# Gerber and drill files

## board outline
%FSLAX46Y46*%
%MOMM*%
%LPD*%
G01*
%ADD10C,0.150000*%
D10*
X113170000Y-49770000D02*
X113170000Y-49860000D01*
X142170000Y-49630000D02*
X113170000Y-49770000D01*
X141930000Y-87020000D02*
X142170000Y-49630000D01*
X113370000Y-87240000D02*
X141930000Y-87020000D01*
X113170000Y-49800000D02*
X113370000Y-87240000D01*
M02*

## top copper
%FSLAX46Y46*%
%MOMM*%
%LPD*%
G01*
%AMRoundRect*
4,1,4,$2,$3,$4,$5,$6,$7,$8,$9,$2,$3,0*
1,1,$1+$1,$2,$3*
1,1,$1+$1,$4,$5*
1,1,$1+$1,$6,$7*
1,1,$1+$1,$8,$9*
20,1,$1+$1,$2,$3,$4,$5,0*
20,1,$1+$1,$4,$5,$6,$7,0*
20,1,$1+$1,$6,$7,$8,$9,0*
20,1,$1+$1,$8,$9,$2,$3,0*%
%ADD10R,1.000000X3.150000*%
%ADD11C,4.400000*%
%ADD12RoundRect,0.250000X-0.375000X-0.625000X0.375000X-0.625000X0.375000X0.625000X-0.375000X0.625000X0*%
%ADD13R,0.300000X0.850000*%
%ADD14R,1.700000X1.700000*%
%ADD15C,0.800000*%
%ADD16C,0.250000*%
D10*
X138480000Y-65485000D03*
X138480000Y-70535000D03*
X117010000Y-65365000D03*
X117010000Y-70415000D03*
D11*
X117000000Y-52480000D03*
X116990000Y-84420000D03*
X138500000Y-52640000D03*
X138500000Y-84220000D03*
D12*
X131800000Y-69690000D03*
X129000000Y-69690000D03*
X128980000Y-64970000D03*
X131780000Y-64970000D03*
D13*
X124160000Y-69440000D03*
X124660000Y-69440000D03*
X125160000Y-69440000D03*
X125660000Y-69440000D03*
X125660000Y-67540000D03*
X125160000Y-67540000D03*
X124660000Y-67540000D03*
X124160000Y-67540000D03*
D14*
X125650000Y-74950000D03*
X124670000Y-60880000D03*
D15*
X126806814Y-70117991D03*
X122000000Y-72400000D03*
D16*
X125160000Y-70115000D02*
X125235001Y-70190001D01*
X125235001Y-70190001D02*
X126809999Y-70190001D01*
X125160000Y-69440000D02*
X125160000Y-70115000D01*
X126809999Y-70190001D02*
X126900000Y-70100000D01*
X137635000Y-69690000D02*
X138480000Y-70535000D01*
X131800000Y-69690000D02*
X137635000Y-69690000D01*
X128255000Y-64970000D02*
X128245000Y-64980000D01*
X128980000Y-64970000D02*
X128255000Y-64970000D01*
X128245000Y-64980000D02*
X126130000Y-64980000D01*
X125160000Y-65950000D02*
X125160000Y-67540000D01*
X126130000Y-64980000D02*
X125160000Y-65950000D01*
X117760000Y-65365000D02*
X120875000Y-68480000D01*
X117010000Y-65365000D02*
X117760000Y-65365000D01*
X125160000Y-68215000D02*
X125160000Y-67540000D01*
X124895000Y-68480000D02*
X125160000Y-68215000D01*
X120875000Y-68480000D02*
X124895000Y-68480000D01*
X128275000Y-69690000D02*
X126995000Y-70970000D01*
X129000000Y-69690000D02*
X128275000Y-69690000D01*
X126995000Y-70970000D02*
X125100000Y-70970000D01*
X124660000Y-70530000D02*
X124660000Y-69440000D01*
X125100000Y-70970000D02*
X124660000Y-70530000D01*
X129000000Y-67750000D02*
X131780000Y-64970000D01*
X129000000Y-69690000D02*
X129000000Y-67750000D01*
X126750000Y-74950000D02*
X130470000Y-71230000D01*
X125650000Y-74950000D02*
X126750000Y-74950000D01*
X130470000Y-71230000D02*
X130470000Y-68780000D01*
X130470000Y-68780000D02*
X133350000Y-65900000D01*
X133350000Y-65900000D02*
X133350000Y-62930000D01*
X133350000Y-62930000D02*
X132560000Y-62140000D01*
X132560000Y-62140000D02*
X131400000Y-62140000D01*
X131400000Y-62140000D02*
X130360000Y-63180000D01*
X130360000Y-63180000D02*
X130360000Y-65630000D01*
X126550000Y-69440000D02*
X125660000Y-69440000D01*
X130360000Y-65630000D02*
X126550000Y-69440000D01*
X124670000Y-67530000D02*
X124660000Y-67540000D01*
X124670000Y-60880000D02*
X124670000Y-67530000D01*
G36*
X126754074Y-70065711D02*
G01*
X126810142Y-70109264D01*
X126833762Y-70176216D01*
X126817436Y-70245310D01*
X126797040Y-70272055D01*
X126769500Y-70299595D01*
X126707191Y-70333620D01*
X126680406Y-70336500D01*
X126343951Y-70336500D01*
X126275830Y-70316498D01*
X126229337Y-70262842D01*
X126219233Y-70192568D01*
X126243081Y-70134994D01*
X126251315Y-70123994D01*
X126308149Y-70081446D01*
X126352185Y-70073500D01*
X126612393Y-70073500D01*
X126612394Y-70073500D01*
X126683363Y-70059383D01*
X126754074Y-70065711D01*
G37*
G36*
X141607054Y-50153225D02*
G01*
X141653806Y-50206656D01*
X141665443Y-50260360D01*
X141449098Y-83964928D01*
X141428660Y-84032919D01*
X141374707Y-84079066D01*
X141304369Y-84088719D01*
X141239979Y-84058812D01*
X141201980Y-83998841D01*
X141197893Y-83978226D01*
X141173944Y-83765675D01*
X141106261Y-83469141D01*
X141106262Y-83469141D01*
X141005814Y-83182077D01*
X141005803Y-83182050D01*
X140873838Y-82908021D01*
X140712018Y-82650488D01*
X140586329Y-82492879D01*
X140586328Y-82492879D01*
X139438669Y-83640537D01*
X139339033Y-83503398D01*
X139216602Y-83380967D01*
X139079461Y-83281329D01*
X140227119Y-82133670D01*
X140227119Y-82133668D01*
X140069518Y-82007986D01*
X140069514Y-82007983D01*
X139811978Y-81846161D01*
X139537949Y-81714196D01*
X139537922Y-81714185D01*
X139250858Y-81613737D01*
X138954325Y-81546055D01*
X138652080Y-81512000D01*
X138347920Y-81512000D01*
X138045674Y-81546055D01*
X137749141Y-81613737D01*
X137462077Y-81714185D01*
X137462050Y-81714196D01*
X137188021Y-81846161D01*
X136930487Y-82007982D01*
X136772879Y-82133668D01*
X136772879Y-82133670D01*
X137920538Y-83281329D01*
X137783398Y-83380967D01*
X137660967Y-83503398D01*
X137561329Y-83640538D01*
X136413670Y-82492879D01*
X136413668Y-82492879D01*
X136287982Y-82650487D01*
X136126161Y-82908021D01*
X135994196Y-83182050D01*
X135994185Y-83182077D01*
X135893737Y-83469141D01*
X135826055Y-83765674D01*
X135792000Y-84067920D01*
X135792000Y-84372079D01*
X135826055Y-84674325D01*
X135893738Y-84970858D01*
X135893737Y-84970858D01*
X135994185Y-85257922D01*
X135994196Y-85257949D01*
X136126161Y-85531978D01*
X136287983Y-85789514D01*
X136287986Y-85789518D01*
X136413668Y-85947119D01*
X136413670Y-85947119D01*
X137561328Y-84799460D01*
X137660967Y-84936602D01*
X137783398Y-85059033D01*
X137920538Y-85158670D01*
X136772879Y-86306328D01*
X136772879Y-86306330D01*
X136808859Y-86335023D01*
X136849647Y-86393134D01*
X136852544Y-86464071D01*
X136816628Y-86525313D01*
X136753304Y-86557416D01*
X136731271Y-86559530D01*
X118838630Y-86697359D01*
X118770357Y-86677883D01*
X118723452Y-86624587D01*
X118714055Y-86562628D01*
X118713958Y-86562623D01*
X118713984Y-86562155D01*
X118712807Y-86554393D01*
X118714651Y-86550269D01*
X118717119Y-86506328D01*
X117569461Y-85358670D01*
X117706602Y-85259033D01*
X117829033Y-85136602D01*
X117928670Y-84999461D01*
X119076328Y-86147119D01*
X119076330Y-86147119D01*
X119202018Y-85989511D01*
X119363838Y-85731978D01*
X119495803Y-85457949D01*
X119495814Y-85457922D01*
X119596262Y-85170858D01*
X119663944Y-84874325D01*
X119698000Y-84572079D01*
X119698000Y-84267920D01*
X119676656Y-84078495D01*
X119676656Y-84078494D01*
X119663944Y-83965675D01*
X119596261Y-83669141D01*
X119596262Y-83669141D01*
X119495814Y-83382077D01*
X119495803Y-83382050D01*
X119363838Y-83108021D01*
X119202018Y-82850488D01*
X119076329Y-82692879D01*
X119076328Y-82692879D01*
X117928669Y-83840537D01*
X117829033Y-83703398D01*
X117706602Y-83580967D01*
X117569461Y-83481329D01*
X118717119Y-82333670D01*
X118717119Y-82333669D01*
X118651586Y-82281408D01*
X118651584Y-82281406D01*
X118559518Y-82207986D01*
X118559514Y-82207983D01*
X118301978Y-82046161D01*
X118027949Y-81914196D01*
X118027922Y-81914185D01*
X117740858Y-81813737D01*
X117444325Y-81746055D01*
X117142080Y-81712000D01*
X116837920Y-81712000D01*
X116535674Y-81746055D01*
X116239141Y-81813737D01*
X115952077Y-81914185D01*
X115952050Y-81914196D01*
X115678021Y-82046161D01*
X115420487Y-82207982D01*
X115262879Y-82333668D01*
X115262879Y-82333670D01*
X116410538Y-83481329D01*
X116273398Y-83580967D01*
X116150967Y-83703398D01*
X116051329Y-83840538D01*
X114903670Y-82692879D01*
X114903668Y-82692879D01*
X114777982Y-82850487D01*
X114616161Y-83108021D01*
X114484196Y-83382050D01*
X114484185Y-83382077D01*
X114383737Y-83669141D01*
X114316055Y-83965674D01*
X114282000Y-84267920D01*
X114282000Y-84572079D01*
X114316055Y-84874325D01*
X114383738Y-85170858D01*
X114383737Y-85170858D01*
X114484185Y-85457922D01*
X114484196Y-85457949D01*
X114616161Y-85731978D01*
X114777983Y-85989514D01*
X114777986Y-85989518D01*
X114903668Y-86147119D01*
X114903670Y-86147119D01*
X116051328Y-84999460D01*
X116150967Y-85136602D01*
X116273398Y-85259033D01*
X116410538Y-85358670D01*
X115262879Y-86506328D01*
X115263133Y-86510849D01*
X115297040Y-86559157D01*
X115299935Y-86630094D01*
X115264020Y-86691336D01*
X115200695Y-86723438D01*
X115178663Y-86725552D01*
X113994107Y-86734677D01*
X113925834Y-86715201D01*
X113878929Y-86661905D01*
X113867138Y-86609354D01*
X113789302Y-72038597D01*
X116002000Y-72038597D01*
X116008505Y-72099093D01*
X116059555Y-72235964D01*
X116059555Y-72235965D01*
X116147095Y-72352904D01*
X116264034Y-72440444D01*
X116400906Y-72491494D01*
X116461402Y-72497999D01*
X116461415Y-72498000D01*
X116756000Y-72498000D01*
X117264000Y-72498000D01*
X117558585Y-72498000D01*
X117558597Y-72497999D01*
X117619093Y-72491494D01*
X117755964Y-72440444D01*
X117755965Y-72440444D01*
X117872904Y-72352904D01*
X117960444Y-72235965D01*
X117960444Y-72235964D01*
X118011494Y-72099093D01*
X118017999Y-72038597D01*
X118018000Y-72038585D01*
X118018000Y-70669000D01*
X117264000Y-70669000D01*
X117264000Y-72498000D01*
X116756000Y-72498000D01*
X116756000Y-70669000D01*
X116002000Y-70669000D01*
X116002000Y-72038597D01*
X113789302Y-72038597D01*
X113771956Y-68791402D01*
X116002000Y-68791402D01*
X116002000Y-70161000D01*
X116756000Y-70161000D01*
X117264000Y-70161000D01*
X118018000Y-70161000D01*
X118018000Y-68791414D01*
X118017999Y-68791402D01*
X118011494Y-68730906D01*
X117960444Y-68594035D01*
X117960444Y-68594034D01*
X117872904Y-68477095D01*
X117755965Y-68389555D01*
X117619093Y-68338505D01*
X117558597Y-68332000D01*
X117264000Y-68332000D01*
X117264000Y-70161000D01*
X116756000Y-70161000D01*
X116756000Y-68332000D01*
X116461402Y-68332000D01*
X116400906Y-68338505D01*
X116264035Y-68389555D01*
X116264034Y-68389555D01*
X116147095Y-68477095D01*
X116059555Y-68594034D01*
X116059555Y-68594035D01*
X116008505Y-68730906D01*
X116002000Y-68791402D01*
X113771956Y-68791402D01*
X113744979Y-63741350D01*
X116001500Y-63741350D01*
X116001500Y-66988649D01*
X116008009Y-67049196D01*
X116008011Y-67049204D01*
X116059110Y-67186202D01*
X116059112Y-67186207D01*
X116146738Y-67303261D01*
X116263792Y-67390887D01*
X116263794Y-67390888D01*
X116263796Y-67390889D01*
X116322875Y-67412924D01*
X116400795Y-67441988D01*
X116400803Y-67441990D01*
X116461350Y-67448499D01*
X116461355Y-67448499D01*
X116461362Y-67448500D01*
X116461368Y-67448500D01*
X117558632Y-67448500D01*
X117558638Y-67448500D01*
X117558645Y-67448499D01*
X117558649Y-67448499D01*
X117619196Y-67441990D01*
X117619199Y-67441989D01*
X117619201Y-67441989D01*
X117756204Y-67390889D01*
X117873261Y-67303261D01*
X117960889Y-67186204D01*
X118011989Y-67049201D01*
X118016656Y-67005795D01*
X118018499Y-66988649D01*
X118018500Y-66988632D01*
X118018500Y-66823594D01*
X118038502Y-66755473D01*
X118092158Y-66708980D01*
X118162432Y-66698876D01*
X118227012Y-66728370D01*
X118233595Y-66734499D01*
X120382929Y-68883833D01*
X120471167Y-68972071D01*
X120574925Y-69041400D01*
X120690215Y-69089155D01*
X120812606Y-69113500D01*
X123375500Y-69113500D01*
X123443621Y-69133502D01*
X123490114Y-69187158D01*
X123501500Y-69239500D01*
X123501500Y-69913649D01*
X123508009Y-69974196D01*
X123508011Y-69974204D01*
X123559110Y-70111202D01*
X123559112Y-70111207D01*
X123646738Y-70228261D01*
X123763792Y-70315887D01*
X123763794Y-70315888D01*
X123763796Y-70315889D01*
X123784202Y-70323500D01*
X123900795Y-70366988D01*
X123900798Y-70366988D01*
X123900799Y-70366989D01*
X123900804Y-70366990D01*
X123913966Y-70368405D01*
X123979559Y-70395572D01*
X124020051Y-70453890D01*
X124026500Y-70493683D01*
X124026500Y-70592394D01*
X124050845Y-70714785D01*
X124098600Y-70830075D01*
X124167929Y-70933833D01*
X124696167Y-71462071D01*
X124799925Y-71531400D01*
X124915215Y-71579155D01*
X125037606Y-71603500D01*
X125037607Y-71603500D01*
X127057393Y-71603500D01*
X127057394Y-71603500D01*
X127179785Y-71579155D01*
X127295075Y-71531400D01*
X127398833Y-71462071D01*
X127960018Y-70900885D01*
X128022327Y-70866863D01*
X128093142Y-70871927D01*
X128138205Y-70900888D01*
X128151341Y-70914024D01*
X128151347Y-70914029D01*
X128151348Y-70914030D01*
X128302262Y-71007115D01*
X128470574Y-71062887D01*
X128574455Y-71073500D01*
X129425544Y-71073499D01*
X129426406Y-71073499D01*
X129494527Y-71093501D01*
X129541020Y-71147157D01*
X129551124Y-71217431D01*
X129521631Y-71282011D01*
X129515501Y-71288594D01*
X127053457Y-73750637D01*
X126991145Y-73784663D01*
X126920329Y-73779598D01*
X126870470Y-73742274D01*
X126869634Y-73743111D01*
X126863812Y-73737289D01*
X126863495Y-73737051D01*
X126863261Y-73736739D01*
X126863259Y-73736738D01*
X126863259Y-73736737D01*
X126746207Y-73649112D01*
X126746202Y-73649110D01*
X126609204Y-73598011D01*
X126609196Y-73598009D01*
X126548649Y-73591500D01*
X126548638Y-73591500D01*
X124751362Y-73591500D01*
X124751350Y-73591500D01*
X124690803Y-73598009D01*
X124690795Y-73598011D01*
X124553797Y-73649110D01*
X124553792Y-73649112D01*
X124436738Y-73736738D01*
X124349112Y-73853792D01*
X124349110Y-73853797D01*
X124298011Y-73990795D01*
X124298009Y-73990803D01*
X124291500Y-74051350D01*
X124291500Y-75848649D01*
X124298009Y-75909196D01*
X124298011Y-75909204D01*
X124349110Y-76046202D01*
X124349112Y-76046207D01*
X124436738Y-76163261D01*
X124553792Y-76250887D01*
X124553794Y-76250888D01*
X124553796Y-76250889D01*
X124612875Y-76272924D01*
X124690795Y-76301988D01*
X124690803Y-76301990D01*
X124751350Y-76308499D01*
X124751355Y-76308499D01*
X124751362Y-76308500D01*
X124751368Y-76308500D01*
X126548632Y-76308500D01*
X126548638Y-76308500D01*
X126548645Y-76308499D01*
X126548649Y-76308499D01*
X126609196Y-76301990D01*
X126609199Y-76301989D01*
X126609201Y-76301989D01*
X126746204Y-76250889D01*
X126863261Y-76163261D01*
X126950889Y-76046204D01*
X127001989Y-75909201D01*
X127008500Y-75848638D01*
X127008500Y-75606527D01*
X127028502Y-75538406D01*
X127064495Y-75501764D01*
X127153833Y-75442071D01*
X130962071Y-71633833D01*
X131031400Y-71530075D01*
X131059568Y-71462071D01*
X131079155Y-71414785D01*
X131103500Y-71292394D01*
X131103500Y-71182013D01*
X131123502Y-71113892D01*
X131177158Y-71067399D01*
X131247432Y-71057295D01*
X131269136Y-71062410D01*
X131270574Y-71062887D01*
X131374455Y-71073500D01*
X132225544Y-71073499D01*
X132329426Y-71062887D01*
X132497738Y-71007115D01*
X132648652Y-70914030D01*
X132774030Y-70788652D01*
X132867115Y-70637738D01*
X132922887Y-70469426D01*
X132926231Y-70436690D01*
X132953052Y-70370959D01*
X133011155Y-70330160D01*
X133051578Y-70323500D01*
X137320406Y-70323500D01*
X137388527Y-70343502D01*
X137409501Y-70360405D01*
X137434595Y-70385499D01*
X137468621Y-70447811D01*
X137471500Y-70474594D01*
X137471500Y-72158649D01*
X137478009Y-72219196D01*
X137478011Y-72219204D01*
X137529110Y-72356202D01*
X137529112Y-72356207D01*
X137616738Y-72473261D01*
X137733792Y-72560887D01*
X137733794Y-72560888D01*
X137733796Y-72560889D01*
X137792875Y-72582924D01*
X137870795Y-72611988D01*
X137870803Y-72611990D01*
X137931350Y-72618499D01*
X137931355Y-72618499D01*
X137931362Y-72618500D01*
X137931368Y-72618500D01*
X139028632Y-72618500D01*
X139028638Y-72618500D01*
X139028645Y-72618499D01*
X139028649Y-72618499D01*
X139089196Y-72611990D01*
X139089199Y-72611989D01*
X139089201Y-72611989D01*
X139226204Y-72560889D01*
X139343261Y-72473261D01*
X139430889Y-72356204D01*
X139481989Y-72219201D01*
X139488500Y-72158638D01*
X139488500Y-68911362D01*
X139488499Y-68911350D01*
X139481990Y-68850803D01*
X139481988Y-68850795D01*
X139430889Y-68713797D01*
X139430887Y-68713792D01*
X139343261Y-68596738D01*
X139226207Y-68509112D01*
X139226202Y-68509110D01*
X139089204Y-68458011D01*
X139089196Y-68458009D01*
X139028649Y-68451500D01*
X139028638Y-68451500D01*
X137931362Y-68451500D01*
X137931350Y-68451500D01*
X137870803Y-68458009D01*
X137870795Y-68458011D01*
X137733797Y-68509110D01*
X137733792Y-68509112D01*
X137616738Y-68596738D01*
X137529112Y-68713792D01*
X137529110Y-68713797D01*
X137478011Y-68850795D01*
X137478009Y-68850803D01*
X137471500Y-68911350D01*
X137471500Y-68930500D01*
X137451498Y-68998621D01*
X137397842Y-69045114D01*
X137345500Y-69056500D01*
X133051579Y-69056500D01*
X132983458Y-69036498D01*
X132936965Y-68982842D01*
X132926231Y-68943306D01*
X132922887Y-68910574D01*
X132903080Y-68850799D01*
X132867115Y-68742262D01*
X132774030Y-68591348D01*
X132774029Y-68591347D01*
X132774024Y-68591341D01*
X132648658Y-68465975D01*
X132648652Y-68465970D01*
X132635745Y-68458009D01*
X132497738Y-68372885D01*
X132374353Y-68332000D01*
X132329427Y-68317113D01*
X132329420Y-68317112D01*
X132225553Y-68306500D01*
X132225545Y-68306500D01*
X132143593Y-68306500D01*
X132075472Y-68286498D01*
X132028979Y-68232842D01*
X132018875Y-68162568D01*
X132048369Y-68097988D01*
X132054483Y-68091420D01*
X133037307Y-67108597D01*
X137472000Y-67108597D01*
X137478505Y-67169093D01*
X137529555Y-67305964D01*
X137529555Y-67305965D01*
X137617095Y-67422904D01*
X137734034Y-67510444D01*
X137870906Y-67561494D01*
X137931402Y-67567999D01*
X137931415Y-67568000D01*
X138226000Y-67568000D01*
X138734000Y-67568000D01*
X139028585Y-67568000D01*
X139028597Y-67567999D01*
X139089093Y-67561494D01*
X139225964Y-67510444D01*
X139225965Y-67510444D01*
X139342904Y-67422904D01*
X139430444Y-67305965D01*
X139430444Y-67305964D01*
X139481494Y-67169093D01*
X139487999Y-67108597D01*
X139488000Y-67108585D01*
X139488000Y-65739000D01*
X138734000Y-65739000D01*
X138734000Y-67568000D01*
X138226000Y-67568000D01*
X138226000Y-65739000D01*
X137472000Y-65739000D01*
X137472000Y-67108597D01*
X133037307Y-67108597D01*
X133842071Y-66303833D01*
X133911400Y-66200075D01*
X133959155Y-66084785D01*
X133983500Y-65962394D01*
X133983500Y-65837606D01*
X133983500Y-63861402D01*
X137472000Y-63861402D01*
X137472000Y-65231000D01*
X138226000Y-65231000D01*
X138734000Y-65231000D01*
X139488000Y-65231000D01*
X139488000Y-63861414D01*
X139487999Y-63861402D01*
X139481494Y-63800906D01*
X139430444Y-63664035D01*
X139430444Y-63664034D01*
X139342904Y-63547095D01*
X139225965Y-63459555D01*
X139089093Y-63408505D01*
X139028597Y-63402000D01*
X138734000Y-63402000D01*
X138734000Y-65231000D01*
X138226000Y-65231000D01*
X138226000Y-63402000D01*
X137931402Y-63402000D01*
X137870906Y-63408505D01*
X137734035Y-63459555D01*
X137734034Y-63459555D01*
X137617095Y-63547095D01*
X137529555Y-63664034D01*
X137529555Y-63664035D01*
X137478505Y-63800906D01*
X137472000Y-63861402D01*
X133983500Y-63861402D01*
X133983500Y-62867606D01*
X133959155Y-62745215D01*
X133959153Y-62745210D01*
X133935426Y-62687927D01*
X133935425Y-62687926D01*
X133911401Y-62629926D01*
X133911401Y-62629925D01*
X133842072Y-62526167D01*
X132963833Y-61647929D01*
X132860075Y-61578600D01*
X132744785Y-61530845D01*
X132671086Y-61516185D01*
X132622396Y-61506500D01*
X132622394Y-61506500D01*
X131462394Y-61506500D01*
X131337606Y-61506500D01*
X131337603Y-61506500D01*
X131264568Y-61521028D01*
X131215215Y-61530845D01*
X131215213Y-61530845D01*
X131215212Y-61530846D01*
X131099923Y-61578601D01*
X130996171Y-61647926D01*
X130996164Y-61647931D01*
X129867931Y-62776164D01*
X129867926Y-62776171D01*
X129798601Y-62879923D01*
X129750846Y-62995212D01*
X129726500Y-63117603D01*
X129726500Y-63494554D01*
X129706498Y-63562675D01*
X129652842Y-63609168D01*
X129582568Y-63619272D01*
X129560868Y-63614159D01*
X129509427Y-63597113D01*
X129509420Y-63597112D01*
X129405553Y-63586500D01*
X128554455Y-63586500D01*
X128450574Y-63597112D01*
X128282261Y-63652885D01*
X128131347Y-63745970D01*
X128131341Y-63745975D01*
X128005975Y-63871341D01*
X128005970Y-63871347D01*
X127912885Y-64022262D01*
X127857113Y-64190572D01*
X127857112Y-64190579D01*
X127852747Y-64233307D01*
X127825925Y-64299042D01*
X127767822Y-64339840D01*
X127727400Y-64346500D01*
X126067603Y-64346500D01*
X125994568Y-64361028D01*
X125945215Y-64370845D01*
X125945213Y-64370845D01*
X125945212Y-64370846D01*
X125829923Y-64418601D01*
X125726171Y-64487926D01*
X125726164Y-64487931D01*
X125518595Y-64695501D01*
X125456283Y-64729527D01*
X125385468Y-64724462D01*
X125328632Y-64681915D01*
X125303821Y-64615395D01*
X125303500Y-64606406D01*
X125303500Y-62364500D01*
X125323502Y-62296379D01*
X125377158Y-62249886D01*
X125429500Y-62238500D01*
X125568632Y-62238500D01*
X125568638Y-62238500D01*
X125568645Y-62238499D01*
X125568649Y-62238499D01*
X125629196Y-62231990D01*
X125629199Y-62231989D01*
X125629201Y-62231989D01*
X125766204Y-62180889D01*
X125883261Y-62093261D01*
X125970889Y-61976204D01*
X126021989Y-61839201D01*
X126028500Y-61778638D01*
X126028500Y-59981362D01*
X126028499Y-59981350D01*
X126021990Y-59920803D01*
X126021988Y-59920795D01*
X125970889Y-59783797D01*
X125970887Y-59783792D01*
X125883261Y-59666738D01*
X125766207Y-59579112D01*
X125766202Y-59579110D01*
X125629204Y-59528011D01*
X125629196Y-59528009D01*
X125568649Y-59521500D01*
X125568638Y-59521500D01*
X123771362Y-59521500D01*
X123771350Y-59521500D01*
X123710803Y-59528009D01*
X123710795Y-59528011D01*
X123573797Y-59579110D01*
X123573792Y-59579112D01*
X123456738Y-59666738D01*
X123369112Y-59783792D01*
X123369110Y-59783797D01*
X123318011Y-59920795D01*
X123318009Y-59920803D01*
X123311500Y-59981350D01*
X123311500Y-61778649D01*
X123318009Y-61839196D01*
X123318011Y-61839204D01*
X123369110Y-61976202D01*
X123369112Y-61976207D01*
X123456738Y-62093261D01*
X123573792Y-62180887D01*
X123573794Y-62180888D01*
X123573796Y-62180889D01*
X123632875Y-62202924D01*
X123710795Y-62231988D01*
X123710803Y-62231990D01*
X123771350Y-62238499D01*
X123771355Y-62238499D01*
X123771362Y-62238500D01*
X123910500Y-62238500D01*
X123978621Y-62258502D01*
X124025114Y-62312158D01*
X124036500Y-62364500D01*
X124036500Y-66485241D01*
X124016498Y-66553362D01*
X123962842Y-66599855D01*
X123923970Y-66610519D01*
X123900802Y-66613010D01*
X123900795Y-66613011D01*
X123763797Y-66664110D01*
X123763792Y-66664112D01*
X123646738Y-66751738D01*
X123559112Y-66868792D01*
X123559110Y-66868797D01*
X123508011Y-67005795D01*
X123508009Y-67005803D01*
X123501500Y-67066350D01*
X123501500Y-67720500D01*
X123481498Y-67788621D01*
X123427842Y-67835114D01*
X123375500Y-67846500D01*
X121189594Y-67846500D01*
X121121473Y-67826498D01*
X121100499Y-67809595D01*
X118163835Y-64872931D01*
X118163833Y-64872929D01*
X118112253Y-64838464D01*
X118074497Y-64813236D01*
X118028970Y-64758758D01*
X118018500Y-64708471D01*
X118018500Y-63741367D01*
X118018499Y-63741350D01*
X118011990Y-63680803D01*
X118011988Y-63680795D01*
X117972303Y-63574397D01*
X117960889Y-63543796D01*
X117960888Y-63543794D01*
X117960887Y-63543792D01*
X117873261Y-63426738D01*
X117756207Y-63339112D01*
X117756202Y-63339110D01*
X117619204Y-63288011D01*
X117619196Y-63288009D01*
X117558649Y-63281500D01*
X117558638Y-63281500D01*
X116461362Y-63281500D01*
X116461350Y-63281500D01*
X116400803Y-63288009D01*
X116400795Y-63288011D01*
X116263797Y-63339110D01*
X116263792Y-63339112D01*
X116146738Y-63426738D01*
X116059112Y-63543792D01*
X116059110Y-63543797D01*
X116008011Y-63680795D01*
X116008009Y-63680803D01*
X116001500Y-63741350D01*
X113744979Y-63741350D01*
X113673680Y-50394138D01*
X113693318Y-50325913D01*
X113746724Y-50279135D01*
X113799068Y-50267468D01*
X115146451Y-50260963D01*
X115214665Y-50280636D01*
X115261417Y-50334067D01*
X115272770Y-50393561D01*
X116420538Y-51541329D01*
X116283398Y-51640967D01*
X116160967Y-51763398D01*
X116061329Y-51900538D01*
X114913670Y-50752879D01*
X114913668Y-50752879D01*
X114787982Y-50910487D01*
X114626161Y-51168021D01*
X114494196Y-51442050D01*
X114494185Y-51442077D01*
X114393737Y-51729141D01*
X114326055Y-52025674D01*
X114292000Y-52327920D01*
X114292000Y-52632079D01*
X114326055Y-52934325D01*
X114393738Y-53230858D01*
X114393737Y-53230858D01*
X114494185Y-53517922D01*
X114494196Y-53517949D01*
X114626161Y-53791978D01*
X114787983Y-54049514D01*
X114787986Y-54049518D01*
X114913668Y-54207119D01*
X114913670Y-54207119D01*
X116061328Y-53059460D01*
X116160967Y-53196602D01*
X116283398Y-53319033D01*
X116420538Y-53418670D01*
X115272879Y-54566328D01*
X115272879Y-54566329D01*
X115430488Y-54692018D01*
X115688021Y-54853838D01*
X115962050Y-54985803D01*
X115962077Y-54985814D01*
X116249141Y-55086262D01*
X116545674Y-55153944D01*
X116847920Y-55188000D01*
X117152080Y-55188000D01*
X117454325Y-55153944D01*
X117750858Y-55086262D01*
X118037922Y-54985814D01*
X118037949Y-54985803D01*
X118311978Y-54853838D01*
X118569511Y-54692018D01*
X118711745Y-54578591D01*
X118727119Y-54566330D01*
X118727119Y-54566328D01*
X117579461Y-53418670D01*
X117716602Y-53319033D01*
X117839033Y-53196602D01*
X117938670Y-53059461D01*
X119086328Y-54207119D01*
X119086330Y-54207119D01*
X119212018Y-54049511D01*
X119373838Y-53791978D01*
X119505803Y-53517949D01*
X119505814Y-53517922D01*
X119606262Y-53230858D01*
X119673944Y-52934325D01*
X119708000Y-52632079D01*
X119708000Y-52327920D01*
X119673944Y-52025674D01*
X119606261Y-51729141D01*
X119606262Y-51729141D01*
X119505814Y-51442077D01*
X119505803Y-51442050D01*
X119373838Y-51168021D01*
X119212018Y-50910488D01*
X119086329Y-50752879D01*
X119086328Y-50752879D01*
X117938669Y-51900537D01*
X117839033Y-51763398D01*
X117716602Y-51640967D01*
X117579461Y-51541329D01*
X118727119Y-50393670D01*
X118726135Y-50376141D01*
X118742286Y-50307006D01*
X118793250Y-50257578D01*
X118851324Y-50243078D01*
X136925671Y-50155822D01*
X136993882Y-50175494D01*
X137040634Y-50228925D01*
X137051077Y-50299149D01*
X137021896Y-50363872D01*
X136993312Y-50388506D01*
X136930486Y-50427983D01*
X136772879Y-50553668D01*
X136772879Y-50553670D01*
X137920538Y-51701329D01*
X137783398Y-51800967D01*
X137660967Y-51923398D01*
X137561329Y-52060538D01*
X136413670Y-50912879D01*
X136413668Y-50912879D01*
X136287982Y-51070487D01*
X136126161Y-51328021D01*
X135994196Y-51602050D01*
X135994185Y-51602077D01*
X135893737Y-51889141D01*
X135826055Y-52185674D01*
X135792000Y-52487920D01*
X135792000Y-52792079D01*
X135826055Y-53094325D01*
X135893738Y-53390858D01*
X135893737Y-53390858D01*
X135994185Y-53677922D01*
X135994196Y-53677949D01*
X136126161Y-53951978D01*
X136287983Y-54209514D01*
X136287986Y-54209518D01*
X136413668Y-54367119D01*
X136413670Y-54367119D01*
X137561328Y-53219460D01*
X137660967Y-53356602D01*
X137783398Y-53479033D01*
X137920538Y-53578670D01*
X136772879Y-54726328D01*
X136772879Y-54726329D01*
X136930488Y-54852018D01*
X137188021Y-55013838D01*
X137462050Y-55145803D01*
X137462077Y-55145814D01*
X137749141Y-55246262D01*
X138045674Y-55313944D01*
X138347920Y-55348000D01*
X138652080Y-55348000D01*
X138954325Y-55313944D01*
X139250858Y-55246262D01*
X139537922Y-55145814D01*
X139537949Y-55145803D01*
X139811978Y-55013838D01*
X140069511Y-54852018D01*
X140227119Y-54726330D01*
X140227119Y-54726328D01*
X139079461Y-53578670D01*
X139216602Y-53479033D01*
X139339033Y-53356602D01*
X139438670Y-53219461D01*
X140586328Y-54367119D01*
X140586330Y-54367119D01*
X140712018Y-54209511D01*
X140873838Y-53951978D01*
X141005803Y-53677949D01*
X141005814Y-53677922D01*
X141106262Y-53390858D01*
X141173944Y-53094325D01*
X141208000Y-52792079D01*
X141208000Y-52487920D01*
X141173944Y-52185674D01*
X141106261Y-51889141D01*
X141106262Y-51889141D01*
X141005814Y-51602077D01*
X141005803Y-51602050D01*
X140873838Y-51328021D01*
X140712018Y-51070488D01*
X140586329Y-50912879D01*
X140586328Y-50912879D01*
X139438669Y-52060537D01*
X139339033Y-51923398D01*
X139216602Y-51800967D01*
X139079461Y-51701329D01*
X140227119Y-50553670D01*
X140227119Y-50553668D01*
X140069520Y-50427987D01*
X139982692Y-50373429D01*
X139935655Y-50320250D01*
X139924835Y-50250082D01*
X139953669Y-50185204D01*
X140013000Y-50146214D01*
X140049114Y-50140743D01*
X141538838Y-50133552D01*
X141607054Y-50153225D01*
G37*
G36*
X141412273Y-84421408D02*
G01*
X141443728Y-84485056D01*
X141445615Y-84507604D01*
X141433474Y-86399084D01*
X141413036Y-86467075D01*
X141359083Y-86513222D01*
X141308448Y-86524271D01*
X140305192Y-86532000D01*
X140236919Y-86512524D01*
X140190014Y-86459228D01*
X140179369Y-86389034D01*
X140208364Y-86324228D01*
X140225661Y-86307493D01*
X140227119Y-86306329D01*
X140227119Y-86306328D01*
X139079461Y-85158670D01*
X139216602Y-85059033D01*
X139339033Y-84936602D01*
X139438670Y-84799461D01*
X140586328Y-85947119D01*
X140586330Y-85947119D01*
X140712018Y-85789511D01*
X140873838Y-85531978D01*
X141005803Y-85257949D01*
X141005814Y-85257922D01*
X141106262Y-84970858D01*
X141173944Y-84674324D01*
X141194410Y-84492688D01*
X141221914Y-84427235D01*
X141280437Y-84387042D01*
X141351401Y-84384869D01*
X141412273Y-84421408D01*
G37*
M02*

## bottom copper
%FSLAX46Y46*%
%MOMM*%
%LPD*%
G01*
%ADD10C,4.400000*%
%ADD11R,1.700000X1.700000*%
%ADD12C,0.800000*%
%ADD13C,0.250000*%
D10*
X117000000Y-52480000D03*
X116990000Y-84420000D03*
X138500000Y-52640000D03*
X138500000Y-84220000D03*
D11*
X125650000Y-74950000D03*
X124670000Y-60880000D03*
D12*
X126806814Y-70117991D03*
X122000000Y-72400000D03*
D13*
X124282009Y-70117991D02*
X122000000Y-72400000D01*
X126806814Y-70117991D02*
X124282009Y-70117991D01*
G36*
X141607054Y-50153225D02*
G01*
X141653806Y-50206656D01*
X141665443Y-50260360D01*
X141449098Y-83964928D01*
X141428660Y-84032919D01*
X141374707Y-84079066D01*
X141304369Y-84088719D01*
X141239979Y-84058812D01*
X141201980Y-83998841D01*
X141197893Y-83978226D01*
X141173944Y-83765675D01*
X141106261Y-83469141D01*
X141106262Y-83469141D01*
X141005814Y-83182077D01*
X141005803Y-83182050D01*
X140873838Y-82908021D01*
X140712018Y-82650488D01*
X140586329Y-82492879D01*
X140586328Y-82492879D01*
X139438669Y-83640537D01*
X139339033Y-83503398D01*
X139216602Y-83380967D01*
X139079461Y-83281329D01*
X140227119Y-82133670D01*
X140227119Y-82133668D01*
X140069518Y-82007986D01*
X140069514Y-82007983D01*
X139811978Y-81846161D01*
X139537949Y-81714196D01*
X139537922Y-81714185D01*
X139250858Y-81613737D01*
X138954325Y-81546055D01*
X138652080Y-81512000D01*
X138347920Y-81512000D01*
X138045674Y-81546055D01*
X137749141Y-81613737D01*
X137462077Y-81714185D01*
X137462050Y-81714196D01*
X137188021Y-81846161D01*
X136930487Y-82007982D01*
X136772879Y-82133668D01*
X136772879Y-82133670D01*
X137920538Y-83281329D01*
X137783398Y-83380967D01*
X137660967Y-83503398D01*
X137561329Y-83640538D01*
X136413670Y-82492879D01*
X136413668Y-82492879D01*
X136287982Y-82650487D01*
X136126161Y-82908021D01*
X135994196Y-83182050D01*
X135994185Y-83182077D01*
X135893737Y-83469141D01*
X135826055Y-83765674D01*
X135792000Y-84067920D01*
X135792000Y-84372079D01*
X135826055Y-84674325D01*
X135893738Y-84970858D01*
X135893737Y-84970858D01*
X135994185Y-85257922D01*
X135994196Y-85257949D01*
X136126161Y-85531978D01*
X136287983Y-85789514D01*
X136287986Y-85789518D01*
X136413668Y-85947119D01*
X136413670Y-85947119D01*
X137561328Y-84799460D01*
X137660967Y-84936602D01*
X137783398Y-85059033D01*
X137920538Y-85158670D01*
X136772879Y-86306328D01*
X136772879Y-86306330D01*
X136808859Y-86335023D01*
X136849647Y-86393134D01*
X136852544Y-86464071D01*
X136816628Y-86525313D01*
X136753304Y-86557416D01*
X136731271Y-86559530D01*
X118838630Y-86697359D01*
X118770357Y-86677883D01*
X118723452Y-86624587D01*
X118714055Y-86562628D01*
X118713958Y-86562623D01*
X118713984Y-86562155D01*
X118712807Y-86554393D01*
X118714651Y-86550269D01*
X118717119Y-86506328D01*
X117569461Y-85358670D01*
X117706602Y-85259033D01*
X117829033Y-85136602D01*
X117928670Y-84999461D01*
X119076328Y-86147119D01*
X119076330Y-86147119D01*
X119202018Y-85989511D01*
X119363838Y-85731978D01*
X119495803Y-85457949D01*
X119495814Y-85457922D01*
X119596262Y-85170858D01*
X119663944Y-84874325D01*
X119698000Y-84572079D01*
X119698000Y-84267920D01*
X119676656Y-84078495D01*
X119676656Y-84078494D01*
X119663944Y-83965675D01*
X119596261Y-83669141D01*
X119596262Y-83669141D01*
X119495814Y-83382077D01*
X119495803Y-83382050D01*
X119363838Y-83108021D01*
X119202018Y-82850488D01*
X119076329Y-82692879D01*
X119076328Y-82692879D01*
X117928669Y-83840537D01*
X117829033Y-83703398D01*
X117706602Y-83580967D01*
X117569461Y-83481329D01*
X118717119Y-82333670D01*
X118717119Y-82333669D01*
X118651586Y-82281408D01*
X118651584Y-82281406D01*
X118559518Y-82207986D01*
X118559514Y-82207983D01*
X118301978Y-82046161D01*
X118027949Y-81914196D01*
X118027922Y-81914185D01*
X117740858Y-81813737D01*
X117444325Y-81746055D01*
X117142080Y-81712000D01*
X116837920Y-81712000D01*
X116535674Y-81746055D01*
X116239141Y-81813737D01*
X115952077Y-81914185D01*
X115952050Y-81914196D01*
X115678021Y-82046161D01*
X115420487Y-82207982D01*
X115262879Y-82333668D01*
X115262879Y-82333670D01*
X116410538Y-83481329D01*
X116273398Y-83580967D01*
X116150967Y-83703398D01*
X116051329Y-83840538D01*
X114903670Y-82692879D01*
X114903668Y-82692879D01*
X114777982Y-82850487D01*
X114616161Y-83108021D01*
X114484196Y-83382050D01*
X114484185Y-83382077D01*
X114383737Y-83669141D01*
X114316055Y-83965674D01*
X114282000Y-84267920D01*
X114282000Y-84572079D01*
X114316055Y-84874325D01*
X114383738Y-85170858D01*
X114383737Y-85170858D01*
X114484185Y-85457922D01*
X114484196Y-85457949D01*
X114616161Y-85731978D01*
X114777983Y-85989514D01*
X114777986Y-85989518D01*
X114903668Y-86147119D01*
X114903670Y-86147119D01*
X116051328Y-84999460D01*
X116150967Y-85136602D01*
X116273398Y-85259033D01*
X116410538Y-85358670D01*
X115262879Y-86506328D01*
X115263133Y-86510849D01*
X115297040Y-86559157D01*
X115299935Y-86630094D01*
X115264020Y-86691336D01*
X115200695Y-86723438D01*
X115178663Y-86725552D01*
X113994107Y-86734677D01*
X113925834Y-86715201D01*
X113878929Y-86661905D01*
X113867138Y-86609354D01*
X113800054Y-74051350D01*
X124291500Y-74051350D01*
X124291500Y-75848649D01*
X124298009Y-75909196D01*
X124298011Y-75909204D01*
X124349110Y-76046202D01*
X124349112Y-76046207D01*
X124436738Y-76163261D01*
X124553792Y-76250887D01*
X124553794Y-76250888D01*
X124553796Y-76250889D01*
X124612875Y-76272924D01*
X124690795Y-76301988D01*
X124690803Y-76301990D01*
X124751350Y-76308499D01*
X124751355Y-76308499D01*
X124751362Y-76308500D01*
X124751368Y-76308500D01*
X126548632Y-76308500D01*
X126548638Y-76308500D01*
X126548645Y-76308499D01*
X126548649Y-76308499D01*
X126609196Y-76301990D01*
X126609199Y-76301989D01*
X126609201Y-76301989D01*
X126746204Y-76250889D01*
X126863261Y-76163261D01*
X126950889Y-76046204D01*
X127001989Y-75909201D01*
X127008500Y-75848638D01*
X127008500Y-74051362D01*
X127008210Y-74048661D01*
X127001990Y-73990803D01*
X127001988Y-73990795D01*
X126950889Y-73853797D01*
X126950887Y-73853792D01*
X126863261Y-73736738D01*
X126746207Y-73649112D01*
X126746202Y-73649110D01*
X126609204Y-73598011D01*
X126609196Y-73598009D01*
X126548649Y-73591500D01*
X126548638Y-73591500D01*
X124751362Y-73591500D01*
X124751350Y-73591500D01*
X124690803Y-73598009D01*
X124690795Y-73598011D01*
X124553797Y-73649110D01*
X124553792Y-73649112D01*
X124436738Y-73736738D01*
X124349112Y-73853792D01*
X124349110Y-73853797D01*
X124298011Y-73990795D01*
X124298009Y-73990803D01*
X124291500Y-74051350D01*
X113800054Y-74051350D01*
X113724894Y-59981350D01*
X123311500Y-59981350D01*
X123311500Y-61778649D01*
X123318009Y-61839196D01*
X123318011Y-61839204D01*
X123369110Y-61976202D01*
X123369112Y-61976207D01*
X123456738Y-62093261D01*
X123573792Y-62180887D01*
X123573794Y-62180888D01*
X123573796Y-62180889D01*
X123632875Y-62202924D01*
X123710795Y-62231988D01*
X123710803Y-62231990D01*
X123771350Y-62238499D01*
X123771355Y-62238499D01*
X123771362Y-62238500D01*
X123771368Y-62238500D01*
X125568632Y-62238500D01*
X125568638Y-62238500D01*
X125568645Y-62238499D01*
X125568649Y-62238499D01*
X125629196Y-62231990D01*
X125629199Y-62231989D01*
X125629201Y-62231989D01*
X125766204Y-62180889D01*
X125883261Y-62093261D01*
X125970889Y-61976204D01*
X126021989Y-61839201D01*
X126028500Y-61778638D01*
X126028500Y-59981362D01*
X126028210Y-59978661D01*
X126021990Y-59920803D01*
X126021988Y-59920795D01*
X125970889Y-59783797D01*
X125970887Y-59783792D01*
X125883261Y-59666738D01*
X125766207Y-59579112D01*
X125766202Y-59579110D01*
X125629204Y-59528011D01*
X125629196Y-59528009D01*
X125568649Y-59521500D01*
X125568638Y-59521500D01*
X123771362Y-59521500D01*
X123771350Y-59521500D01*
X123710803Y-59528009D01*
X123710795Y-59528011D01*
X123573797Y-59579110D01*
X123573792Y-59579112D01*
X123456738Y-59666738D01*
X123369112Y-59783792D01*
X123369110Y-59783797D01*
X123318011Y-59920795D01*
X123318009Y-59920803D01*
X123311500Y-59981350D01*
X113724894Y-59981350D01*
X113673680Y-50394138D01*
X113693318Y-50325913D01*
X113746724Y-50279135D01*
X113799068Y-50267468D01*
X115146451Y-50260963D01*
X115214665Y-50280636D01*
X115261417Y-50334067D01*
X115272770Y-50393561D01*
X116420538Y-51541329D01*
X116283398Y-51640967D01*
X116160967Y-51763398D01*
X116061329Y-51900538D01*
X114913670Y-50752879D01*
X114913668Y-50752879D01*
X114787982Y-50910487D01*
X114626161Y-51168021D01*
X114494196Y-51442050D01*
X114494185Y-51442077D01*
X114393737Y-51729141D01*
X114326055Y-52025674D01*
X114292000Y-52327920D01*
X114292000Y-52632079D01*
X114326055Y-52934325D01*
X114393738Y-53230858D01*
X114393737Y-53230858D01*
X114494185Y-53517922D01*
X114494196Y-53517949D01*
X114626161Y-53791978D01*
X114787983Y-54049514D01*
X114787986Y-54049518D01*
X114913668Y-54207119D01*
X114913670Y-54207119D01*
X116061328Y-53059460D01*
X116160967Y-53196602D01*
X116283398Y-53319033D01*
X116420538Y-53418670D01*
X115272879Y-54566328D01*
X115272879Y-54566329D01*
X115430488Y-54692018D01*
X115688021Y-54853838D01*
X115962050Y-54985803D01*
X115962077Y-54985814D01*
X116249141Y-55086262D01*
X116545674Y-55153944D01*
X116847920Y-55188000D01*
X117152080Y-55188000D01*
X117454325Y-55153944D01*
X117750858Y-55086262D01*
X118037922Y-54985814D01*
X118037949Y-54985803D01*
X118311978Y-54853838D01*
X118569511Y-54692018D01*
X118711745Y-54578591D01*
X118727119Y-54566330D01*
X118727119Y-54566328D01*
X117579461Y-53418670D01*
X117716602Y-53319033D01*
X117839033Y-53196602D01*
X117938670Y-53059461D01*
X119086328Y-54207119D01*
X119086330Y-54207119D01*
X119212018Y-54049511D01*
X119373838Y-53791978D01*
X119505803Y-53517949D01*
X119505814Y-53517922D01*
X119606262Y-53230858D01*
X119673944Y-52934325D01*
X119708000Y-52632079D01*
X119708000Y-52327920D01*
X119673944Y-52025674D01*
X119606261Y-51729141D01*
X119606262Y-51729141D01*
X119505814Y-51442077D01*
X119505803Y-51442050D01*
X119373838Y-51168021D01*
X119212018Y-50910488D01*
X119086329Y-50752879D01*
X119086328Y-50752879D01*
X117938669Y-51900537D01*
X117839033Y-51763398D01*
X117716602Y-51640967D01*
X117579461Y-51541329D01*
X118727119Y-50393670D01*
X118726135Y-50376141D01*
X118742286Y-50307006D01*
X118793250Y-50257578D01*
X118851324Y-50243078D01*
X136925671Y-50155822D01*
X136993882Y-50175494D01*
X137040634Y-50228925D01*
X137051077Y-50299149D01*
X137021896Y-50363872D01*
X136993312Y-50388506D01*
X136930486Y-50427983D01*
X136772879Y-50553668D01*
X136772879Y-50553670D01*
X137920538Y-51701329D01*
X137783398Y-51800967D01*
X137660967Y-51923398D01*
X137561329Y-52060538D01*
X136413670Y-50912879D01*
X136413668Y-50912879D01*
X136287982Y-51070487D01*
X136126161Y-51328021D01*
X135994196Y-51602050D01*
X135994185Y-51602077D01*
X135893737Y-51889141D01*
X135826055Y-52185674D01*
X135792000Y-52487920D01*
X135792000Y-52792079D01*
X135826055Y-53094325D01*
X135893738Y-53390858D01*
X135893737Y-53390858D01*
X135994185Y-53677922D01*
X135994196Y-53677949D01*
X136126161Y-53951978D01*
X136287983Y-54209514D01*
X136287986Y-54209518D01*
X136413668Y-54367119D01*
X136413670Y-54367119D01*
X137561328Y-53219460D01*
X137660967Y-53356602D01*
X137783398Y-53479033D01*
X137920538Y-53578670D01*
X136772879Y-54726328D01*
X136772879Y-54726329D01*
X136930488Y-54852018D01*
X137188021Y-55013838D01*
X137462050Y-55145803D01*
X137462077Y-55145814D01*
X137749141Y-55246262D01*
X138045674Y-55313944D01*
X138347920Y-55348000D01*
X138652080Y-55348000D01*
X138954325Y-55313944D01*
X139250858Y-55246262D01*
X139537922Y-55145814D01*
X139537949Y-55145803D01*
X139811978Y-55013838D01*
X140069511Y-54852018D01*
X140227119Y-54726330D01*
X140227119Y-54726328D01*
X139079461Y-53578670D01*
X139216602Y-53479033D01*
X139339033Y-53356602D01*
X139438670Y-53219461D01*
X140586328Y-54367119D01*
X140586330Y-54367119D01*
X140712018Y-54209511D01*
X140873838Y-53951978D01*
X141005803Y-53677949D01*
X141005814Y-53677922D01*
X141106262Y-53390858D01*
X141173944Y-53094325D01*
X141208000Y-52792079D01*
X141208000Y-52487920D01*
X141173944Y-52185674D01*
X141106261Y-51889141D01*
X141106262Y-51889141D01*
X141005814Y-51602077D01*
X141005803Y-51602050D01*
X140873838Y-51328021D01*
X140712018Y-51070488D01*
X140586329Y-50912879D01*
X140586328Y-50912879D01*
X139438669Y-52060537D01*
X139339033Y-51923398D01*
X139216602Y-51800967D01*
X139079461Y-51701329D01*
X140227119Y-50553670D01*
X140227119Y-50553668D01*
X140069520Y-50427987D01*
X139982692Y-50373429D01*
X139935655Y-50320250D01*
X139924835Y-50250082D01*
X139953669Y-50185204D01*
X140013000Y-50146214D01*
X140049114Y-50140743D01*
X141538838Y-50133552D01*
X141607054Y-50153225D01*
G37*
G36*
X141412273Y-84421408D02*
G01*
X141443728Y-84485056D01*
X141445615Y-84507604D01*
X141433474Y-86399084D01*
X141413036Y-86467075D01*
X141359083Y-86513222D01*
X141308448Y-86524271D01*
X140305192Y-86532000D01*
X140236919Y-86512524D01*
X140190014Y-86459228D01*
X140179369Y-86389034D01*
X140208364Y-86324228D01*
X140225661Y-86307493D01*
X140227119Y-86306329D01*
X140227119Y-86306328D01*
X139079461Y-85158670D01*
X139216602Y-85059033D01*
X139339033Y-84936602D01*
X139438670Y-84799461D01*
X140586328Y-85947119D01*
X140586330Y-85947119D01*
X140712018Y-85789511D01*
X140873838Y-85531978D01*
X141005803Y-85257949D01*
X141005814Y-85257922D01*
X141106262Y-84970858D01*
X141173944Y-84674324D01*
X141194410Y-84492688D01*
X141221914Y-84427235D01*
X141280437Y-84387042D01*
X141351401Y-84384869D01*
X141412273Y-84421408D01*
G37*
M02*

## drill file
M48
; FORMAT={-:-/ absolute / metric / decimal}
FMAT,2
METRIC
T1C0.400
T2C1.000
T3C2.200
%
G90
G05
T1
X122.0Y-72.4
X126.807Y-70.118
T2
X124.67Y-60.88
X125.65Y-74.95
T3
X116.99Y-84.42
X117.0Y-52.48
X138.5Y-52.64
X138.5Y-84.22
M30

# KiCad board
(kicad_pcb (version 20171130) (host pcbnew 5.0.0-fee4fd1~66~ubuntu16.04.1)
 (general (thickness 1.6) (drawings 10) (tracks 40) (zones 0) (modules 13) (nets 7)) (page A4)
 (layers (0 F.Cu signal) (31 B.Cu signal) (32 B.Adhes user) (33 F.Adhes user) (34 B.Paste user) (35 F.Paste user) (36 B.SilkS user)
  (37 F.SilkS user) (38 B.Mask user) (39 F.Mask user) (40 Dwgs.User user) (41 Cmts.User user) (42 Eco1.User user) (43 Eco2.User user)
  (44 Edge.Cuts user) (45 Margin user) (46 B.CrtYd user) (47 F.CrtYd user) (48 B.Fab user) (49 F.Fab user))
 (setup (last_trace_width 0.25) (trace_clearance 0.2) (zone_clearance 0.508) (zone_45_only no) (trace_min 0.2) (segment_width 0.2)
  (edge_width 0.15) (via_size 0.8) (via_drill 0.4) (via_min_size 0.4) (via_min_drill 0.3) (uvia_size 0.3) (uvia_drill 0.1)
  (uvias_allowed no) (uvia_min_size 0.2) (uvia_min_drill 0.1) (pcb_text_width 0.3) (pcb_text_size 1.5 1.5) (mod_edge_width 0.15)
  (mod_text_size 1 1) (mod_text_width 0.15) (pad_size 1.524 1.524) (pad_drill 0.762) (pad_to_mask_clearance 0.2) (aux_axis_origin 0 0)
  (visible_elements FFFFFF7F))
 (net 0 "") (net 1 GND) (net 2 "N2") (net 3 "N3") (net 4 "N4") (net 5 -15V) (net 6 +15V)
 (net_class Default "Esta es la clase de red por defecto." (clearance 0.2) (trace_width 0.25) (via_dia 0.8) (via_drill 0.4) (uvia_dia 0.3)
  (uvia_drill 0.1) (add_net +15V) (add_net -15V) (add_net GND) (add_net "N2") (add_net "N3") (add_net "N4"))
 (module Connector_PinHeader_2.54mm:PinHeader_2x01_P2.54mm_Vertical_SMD (layer F.Cu) (at 138.48 68.01 270)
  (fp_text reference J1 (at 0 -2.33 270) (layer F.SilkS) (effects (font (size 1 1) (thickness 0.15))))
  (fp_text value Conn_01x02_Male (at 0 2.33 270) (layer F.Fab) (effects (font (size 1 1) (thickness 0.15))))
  (pad 1 smd rect (at -2.525 0 270) (size 3.15 1) (layers F.Cu F.Paste F.Mask) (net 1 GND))
  (pad 2 smd rect (at 2.525 0 270) (size 3.15 1) (layers F.Cu F.Paste F.Mask) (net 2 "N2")))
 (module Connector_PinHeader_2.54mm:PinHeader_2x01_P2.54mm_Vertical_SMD (layer F.Cu) (at 117.01 67.89 90)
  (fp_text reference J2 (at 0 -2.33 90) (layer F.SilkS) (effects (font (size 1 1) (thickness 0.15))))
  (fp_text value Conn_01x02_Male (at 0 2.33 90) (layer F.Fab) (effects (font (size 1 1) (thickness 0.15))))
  (pad 2 smd rect (at 2.525 0 90) (size 3.15 1) (layers F.Cu F.Paste F.Mask) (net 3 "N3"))
  (pad 1 smd rect (at -2.525 0 90) (size 3.15 1) (layers F.Cu F.Paste F.Mask) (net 1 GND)))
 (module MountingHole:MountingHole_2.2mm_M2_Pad (layer F.Cu) (at 117 52.48)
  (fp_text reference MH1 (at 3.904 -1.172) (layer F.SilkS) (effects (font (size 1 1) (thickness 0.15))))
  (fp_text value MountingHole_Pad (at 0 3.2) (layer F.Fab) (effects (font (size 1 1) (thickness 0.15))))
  (pad 1 thru_hole circle (at 0 0) (size 4.4 4.4) (drill 2.2) (layers *.Cu *.Mask) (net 1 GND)))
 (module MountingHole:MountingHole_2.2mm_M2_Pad (layer F.Cu) (at 116.99 84.42)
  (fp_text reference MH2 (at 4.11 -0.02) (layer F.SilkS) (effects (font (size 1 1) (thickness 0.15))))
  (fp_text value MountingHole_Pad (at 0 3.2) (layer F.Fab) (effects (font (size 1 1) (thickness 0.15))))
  (pad 1 thru_hole circle (at 0 0) (size 4.4 4.4) (drill 2.2) (layers *.Cu *.Mask) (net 1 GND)))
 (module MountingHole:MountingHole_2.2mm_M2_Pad (layer F.Cu) (at 138.5 52.64)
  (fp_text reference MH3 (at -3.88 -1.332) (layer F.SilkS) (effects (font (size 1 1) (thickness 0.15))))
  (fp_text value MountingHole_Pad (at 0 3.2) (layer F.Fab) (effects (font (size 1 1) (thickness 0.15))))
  (pad 1 thru_hole circle (at 0 0) (size 4.4 4.4) (drill 2.2) (layers *.Cu *.Mask) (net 1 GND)))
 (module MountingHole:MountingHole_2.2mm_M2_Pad (layer F.Cu) (at 138.5 84.22)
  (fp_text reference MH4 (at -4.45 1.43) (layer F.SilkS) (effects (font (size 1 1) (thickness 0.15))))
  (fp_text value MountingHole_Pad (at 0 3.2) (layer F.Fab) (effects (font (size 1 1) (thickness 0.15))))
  (pad 1 thru_hole circle (at 0 0) (size 4.4 4.4) (drill 2.2) (layers *.Cu *.Mask) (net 1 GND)))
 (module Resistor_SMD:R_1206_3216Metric (layer F.Cu) (at 130.4 69.69)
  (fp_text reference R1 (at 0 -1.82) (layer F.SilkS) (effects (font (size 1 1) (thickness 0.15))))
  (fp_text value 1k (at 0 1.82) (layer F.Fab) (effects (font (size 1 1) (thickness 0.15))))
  (pad 2 smd roundrect (at 1.4 0) (size 1.25 1.75) (layers F.Cu F.Paste F.Mask) (roundrect_rratio 0.2) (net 2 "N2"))
  (pad 1 smd roundrect (at -1.4 0) (size 1.25 1.75) (layers F.Cu F.Paste F.Mask) (roundrect_rratio 0.2) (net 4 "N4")))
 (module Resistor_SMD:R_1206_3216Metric (layer F.Cu) (at 130.38 64.97)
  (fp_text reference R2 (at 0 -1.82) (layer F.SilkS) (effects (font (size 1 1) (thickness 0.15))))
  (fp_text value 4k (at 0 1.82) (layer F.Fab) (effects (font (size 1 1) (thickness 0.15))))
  (pad 1 smd roundrect (at -1.4 0) (size 1.25 1.75) (layers F.Cu F.Paste F.Mask) (roundrect_rratio 0.2) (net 3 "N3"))
  (pad 2 smd roundrect (at 1.4 0) (size 1.25 1.75) (layers F.Cu F.Paste F.Mask) (roundrect_rratio 0.2) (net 4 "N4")))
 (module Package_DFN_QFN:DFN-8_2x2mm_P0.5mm (layer F.Cu) (at 124.91 68.49 90)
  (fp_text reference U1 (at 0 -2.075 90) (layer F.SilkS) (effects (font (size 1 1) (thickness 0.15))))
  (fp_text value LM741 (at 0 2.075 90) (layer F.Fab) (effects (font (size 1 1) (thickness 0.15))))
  (pad 1 smd rect (at -0.95 -0.75 90) (size 0.85 0.3) (layers F.Cu F.Paste F.Mask))
  (pad 2 smd rect (at -0.95 -0.25 90) (size 0.85 0.3) (layers F.Cu F.Paste F.Mask) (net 4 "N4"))
  (pad 3 smd rect (at -0.95 0.25 90) (size 0.85 0.3) (layers F.Cu F.Paste F.Mask) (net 1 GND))
  (pad 4 smd rect (at -0.95 0.75 90) (size 0.85 0.3) (layers F.Cu F.Paste F.Mask) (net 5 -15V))
  (pad 5 smd rect (at 0.95 0.75 90) (size 0.85 0.3) (layers F.Cu F.Paste F.Mask))
  (pad 6 smd rect (at 0.95 0.25 90) (size 0.85 0.3) (layers F.Cu F.Paste F.Mask) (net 3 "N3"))
  (pad 7 smd rect (at 0.95 -0.25 90) (size 0.85 0.3) (layers F.Cu F.Paste F.Mask) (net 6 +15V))
  (pad 8 smd rect (at 0.95 -0.75 90) (size 0.85 0.3) (layers F.Cu F.Paste F.Mask)))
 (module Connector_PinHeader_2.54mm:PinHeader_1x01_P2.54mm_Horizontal (layer F.Cu) (at 125.65 74.95 270)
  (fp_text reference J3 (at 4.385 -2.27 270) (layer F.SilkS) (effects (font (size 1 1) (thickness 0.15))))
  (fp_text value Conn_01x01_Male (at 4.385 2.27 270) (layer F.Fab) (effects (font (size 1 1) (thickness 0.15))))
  (pad 1 thru_hole rect (at 0 0 270) (size 1.7 1.7) (drill 1) (layers *.Cu *.Mask) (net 5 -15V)))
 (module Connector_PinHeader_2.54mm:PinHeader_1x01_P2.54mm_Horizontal (layer F.Cu) (at 124.67 60.88 90)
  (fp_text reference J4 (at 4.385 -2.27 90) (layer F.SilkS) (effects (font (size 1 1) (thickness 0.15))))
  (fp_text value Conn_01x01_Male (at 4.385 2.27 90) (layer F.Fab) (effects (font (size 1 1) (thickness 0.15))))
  (pad 1 thru_hole rect (at 0 0 90) (size 1.7 1.7) (drill 1) (layers *.Cu *.Mask) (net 6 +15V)))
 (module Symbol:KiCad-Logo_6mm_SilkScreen (layer F.Cu) (at 134.4 57.6)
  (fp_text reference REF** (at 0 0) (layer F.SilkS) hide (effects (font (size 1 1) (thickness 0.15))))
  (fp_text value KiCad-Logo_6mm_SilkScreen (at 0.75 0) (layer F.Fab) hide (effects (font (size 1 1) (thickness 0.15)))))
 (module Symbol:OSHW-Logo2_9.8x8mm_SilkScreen (layer F.Cu) (at 118.4 78.2)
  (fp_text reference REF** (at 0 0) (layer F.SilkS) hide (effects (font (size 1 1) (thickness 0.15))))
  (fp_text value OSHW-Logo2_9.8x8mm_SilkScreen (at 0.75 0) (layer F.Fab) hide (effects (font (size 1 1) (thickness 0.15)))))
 (gr_line (start 113.17 49.77) (end 113.17 49.86) (layer Edge.Cuts) (width 0.15))
 (gr_line (start 142.17 49.63) (end 113.17 49.77) (layer Edge.Cuts) (width 0.15))
 (gr_line (start 141.93 87.02) (end 142.17 49.63) (layer Edge.Cuts) (width 0.15))
 (gr_line (start 113.37 87.24) (end 141.93 87.02) (layer Edge.Cuts) (width 0.15))
 (gr_line (start 113.17 49.8) (end 113.37 87.24) (layer Edge.Cuts) (width 0.15))
 (segment (start 125.16 70.115) (end 125.235001 70.190001) (width 0.25) (layer F.Cu) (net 1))
 (segment (start 125.235001 70.190001) (end 126.809999 70.190001) (width 0.25) (layer F.Cu) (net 1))
 (via (at 126.806814 70.117991) (size 0.8) (drill 0.4) (layers F.Cu B.Cu) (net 1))
 (segment (start 125.16 69.44) (end 125.16 70.115) (width 0.25) (layer F.Cu) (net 1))
 (segment (start 126.809999 70.190001) (end 126.9 70.1) (width 0.25) (layer F.Cu) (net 1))
 (via (at 122 72.4) (size 0.8) (drill 0.4) (layers F.Cu B.Cu) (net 1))
 (segment (start 124.282009 70.117991) (end 122 72.4) (width 0.25) (layer B.Cu) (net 1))
 (segment (start 126.806814 70.117991) (end 124.282009 70.117991) (width 0.25) (layer B.Cu) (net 1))
 (segment (start 137.635 69.69) (end 138.48 70.535) (width 0.25) (layer F.Cu) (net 2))
 (segment (start 131.8 69.69) (end 137.635 69.69) (width 0.25) (layer F.Cu) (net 2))
 (segment (start 128.255 64.97) (end 128.245 64.98) (width 0.25) (layer F.Cu) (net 3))
 (segment (start 128.98 64.97) (end 128.255 64.97) (width 0.25) (layer F.Cu) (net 3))
 (segment (start 128.245 64.98) (end 126.13 64.98) (width 0.25) (layer F.Cu) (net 3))
 (segment (start 125.16 65.95) (end 125.16 67.54) (width 0.25) (layer F.Cu) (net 3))
 (segment (start 126.13 64.98) (end 125.16 65.95) (width 0.25) (layer F.Cu) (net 3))
 (segment (start 117.76 65.365) (end 120.875 68.48) (width 0.25) (layer F.Cu) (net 3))
 (segment (start 117.01 65.365) (end 117.76 65.365) (width 0.25) (layer F.Cu) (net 3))
 (segment (start 125.16 68.215) (end 125.16 67.54) (width 0.25) (layer F.Cu) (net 3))
 (segment (start 124.895 68.48) (end 125.16 68.215) (width 0.25) (layer F.Cu) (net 3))
 (segment (start 120.875 68.48) (end 124.895 68.48) (width 0.25) (layer F.Cu) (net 3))
 (segment (start 128.275 69.69) (end 126.995 70.97) (width 0.25) (layer F.Cu) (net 4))
 (segment (start 129 69.69) (end 128.275 69.69) (width 0.25) (layer F.Cu) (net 4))
 (segment (start 126.995 70.97) (end 125.1 70.97) (width 0.25) (layer F.Cu) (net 4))
 (segment (start 124.66 70.53) (end 124.66 69.44) (width 0.25) (layer F.Cu) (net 4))
 (segment (start 125.1 70.97) (end 124.66 70.53) (width 0.25) (layer F.Cu) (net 4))
 (segment (start 129 67.75) (end 131.78 64.97) (width 0.25) (layer F.Cu) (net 4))
 (segment (start 129 69.69) (end 129 67.75) (width 0.25) (layer F.Cu) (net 4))
 (segment (start 126.75 74.95) (end 130.47 71.23) (width 0.25) (layer F.Cu) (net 5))
 (segment (start 125.65 74.95) (end 126.75 74.95) (width 0.25) (layer F.Cu) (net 5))
 (segment (start 130.47 71.23) (end 130.47 68.78) (width 0.25) (layer F.Cu) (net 5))
 (segment (start 130.47 68.78) (end 133.35 65.9) (width 0.25) (layer F.Cu) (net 5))
 (segment (start 133.35 65.9) (end 133.35 62.93) (width 0.25) (layer F.Cu) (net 5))
 (segment (start 133.35 62.93) (end 132.56 62.14) (width 0.25) (layer F.Cu) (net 5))
 (segment (start 132.56 62.14) (end 131.4 62.14) (width 0.25) (layer F.Cu) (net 5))
 (segment (start 131.4 62.14) (end 130.36 63.18) (width 0.25) (layer F.Cu) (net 5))
 (segment (start 130.36 63.18) (end 130.36 65.63) (width 0.25) (layer F.Cu) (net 5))
 (segment (start 126.55 69.44) (end 125.66 69.44) (width 0.25) (layer F.Cu) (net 5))
 (segment (start 130.36 65.63) (end 126.55 69.44) (width 0.25) (layer F.Cu) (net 5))
 (segment (start 124.67 67.53) (end 124.66 67.54) (width 0.25) (layer F.Cu) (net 6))
 (segment (start 124.67 60.88) (end 124.67 67.53) (width 0.25) (layer F.Cu) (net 6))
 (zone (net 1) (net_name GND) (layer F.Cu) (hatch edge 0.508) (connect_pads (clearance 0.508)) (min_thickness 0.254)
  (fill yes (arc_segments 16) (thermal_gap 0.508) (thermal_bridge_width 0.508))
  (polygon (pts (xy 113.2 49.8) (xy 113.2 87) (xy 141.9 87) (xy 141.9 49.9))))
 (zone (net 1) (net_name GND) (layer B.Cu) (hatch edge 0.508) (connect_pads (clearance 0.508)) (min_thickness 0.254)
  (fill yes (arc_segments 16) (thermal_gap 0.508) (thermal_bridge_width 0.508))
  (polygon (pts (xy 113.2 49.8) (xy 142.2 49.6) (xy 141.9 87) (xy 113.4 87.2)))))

